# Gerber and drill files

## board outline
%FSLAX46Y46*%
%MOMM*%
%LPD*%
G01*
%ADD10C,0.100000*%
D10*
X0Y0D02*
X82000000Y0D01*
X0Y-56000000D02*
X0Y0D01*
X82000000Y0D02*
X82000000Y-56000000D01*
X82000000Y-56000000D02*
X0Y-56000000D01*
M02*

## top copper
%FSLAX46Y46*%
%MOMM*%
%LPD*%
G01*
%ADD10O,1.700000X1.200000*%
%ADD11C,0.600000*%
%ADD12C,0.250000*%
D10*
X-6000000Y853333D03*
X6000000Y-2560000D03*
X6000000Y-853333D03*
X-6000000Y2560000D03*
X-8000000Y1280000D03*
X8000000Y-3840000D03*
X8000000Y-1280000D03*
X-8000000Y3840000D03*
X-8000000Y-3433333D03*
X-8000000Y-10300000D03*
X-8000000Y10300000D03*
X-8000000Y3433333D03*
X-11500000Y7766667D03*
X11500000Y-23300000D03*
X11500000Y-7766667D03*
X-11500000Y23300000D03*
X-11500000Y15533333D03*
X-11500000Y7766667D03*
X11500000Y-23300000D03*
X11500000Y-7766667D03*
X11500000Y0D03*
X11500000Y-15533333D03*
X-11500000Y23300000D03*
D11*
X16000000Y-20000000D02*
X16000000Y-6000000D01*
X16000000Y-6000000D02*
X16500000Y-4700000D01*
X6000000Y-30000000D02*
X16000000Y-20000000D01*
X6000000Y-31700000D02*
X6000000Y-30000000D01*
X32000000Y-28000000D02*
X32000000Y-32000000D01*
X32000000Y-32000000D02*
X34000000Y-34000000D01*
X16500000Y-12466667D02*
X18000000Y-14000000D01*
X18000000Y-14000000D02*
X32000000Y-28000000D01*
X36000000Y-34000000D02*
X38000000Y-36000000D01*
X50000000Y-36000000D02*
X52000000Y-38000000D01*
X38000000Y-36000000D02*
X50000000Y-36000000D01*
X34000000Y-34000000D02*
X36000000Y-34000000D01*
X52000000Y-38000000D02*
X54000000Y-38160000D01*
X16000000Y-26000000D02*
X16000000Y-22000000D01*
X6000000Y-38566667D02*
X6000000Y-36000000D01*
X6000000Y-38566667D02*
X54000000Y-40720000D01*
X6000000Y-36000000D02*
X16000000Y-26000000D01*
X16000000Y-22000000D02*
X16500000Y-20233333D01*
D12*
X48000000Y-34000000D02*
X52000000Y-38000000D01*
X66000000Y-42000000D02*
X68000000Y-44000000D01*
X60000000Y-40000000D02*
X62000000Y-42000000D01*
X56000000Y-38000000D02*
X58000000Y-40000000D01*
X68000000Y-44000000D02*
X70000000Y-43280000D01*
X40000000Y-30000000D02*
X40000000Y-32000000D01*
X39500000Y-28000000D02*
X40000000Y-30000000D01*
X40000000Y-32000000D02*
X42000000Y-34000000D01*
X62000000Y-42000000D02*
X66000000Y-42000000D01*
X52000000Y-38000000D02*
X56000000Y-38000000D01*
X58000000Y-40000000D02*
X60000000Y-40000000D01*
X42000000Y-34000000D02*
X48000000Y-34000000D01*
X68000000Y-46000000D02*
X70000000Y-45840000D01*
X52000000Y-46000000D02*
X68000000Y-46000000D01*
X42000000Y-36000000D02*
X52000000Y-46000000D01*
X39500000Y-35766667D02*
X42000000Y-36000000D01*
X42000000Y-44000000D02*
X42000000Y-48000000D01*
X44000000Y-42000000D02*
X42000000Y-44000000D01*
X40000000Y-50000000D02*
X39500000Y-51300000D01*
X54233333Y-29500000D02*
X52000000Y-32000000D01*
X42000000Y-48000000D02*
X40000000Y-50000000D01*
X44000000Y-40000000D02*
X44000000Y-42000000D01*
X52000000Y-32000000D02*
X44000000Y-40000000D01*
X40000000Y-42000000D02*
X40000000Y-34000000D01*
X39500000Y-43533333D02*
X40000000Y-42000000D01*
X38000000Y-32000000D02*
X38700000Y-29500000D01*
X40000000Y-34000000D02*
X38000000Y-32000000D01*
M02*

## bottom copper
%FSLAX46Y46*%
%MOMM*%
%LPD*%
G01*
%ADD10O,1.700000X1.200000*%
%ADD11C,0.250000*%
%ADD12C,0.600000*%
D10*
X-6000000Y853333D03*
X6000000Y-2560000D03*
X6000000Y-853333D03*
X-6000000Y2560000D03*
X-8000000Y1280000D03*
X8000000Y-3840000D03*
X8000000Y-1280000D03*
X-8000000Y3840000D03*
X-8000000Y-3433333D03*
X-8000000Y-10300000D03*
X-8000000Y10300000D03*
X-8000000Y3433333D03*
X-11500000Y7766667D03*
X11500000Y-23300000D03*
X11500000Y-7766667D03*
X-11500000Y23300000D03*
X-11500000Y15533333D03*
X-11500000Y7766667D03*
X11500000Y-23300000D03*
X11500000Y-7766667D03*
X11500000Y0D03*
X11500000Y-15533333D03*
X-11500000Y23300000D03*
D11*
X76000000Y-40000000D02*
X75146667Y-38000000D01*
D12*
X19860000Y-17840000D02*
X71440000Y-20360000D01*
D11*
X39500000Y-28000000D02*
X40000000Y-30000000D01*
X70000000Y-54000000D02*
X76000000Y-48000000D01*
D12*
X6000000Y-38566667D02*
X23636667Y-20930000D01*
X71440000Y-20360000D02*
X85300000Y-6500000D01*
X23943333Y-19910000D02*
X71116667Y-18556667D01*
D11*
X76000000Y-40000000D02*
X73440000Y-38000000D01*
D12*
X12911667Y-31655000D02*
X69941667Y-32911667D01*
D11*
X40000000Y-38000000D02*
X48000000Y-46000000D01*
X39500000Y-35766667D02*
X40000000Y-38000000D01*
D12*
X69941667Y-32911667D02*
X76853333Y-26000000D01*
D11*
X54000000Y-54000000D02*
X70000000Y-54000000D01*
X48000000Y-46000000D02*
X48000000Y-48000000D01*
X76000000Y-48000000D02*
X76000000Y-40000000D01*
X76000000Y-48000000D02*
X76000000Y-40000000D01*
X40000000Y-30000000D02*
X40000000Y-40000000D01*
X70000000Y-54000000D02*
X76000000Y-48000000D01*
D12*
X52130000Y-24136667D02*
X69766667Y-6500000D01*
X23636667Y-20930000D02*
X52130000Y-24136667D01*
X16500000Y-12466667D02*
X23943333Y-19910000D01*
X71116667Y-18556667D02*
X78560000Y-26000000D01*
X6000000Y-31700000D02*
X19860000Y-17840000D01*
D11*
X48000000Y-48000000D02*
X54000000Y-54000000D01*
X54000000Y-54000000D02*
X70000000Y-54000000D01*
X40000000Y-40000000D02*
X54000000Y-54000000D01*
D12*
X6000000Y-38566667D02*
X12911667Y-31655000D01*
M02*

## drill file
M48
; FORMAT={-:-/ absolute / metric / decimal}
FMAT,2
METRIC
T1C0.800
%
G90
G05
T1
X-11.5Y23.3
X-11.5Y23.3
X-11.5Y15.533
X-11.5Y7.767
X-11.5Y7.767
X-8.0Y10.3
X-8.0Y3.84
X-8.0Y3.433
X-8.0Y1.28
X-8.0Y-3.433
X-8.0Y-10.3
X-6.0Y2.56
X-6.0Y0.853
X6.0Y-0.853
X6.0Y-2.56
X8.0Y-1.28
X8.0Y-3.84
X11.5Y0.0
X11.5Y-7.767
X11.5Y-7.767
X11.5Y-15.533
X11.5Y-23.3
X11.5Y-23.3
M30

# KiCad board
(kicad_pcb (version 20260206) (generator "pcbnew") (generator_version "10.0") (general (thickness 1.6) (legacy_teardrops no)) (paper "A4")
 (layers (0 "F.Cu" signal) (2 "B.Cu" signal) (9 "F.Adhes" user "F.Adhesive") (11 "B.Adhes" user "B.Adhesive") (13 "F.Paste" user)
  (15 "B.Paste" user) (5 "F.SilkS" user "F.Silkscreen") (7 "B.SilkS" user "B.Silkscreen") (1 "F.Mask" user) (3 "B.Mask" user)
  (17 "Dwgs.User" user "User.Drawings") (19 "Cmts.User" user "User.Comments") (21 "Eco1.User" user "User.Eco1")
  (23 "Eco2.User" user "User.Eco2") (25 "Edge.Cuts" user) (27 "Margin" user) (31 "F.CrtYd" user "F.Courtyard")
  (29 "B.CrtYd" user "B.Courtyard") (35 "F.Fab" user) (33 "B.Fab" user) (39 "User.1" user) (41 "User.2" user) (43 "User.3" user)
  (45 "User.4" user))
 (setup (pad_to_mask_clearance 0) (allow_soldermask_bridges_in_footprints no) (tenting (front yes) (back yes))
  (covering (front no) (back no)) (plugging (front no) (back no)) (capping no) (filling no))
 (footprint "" (layer "F.Cu") (at 76 32 90)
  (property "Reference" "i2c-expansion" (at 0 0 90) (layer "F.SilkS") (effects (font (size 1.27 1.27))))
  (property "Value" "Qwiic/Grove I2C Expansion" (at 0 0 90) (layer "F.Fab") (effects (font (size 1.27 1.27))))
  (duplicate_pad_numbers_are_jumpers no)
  (pad "GND" thru_hole oval (at 32.853333 -82) (size 1.7 1.2) (drill 0.8) (layers "*.Cu") (remove_unused_layers no) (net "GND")
   (thermal_bridge_angle 45))
  (pad "SCL" thru_hole oval (at 29.44 -70) (size 1.7 1.2) (drill 0.8) (layers "*.Cu") (remove_unused_layers no) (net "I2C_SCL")
   (thermal_bridge_angle 45))
  (pad "SDA" thru_hole oval (at 31.146667 -70) (size 1.7 1.2) (drill 0.8) (layers "*.Cu") (remove_unused_layers no) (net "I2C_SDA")
   (thermal_bridge_angle 45))
  (pad "VCC" thru_hole oval (at 34.56 -82) (size 1.7 1.2) (drill 0.8) (layers "*.Cu") (remove_unused_layers no) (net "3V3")
   (thermal_bridge_angle 45)))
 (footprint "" (layer "F.Cu") (at 62 42)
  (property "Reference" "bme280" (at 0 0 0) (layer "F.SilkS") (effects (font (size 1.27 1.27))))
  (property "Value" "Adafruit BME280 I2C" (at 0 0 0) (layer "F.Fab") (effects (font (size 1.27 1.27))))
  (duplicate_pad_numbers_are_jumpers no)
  (pad "GND" thru_hole oval (at -70 -43.28) (size 1.7 1.2) (drill 0.8) (layers "*.Cu") (remove_unused_layers no) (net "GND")
   (thermal_bridge_angle 45))
  (pad "SCL" thru_hole oval (at -54 -38.16) (size 1.7 1.2) (drill 0.8) (layers "*.Cu") (remove_unused_layers no) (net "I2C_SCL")
   (thermal_bridge_angle 45))
  (pad "SDA" thru_hole oval (at -54 -40.72) (size 1.7 1.2) (drill 0.8) (layers "*.Cu") (remove_unused_layers no) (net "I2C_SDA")
   (thermal_bridge_angle 45))
  (pad "VCC" thru_hole oval (at -70 -45.84) (size 1.7 1.2) (drill 0.8) (layers "*.Cu") (remove_unused_layers no) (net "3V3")
   (thermal_bridge_angle 45)))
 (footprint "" (layer "F.Cu") (at 14 42)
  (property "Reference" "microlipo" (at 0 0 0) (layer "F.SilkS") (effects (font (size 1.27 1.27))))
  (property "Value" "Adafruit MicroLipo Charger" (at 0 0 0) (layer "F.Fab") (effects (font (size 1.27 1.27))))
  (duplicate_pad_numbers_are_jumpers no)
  (pad "B+" thru_hole oval (at -22 -38.566667) (size 1.7 1.2) (drill 0.8) (layers "*.Cu") (remove_unused_layers no)
   (thermal_bridge_angle 45))
  (pad "B-" thru_hole oval (at -22 -31.7) (size 1.7 1.2) (drill 0.8) (layers "*.Cu") (remove_unused_layers no) (thermal_bridge_angle 45))
  (pad "OUT+" thru_hole oval (at -22 -52.3) (size 1.7 1.2) (drill 0.8) (layers "*.Cu") (remove_unused_layers no) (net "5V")
   (thermal_bridge_angle 45))
  (pad "OUT-" thru_hole oval (at -22 -45.433333) (size 1.7 1.2) (drill 0.8) (layers "*.Cu") (remove_unused_layers no) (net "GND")
   (thermal_bridge_angle 45)))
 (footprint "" (layer "F.Cu") (at 62 18 90)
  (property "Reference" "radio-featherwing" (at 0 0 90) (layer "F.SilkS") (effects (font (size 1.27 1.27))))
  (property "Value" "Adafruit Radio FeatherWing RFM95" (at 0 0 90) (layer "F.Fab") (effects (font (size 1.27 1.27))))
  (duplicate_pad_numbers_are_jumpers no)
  (pad "GND" thru_hole oval (at 25.766667 -73.5) (size 1.7 1.2) (drill 0.8) (layers "*.Cu") (remove_unused_layers no) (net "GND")
   (thermal_bridge_angle 45))
  (pad "RX" thru_hole oval (at -5.3 -50.5) (size 1.7 1.2) (drill 0.8) (layers "*.Cu") (remove_unused_layers no) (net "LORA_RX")
   (thermal_bridge_angle 45))
  (pad "TX" thru_hole oval (at 10.233333 -50.5) (size 1.7 1.2) (drill 0.8) (layers "*.Cu") (remove_unused_layers no) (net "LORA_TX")
   (thermal_bridge_angle 45))
  (pad "VCC" thru_hole oval (at 41.3 -73.5) (size 1.7 1.2) (drill 0.8) (layers "*.Cu") (remove_unused_layers no) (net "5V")
   (thermal_bridge_angle 45)))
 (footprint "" (layer "F.Cu") (at 28 28)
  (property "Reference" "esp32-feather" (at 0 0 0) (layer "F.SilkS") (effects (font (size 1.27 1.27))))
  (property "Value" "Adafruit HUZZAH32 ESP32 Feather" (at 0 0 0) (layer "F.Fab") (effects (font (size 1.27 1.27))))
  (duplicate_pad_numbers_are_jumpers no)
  (pad "3V3" thru_hole oval (at -39.5 -43.533333) (size 1.7 1.2) (drill 0.8) (layers "*.Cu") (remove_unused_layers no) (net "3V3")
   (thermal_bridge_angle 45))
  (pad "GND" thru_hole oval (at -39.5 -35.766667) (size 1.7 1.2) (drill 0.8) (layers "*.Cu") (remove_unused_layers no) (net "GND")
   (thermal_bridge_angle 45))
  (pad "RX" thru_hole oval (at -16.5 -4.7) (size 1.7 1.2) (drill 0.8) (layers "*.Cu") (remove_unused_layers no) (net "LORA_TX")
   (thermal_bridge_angle 45))
  (pad "SCL" thru_hole oval (at -16.5 -20.233333) (size 1.7 1.2) (drill 0.8) (layers "*.Cu") (remove_unused_layers no) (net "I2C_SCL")
   (thermal_bridge_angle 45))
  (pad "SDA" thru_hole oval (at -16.5 -28) (size 1.7 1.2) (drill 0.8) (layers "*.Cu") (remove_unused_layers no) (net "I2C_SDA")
   (thermal_bridge_angle 45))
  (pad "TX" thru_hole oval (at -16.5 -12.466667) (size 1.7 1.2) (drill 0.8) (layers "*.Cu") (remove_unused_layers no) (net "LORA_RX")
   (thermal_bridge_angle 45))
  (pad "VIN" thru_hole oval (at -39.5 -51.3) (size 1.7 1.2) (drill 0.8) (layers "*.Cu") (remove_unused_layers no) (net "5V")
   (thermal_bridge_angle 45)))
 (gr_line (start 0 0) (end 82 0) (stroke (width 0.1) (type default)) (layer "Edge.Cuts"))
 (gr_line (start 0 56) (end 0 0) (stroke (width 0.1) (type default)) (layer "Edge.Cuts"))
 (gr_line (start 82 0) (end 82 56) (stroke (width 0.1) (type default)) (layer "Edge.Cuts"))
 (gr_line (start 82 56) (end 0 56) (stroke (width 0.1) (type default)) (layer "Edge.Cuts"))
 (segment (start 16 20) (end 16 6) (width 0.6) (layer "F.Cu") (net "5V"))
 (segment (start 16 6) (end 16.5 4.7) (width 0.6) (layer "F.Cu") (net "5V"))
 (segment (start 6 30) (end 16 20) (width 0.6) (layer "F.Cu") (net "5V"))
 (segment (start 6 31.7) (end 6 30) (width 0.6) (layer "F.Cu") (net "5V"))
 (segment (start 32 28) (end 32 32) (width 0.6) (layer "F.Cu") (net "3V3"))
 (segment (start 32 32) (end 34 34) (width 0.6) (layer "F.Cu") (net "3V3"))
 (segment (start 16.5 12.466667) (end 18 14) (width 0.6) (layer "F.Cu") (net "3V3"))
 (segment (start 18 14) (end 32 28) (width 0.6) (layer "F.Cu") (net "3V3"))
 (segment (start 36 34) (end 38 36) (width 0.6) (layer "F.Cu") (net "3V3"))
 (segment (start 50 36) (end 52 38) (width 0.6) (layer "F.Cu") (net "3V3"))
 (segment (start 38 36) (end 50 36) (width 0.6) (layer "F.Cu") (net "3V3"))
 (segment (start 34 34) (end 36 34) (width 0.6) (layer "F.Cu") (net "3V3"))
 (segment (start 52 38) (end 54 38.16) (width 0.6) (layer "F.Cu") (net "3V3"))
 (segment (start 16 26) (end 16 22) (width 0.6) (layer "F.Cu") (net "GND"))
 (segment (start 6 38.566667) (end 6 36) (width 0.6) (layer "F.Cu") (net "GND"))
 (segment (start 6 38.566667) (end 54 40.72) (width 0.6) (layer "F.Cu") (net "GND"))
 (segment (start 6 36) (end 16 26) (width 0.6) (layer "F.Cu") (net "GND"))
 (segment (start 16 22) (end 16.5 20.233333) (width 0.6) (layer "F.Cu") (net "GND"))
 (segment (start 48 34) (end 52 38) (width 0.25) (layer "F.Cu") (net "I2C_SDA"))
 (segment (start 66 42) (end 68 44) (width 0.25) (layer "F.Cu") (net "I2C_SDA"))
 (segment (start 60 40) (end 62 42) (width 0.25) (layer "F.Cu") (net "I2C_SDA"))
 (segment (start 56 38) (end 58 40) (width 0.25) (layer "F.Cu") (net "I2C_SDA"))
 (segment (start 68 44) (end 70 43.28) (width 0.25) (layer "F.Cu") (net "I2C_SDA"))
 (segment (start 40 30) (end 40 32) (width 0.25) (layer "F.Cu") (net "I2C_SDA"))
 (segment (start 39.5 28) (end 40 30) (width 0.25) (layer "F.Cu") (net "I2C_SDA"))
 (segment (start 40 32) (end 42 34) (width 0.25) (layer "F.Cu") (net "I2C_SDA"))
 (segment (start 62 42) (end 66 42) (width 0.25) (layer "F.Cu") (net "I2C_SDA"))
 (segment (start 52 38) (end 56 38) (width 0.25) (layer "F.Cu") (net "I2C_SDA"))
 (segment (start 58 40) (end 60 40) (width 0.25) (layer "F.Cu") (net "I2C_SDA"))
 (segment (start 42 34) (end 48 34) (width 0.25) (layer "F.Cu") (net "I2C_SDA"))
 (segment (start 68 46) (end 70 45.84) (width 0.25) (layer "F.Cu") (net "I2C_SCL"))
 (segment (start 52 46) (end 68 46) (width 0.25) (layer "F.Cu") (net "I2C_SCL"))
 (segment (start 42 36) (end 52 46) (width 0.25) (layer "F.Cu") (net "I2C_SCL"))
 (segment (start 39.5 35.766667) (end 42 36) (width 0.25) (layer "F.Cu") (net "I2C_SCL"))
 (segment (start 76 40) (end 75.146667 38) (width 0.25) (layer "B.Cu") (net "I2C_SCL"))
 (segment (start 19.86 17.84) (end 71.44 20.36) (width 0.6) (layer "B.Cu") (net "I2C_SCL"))
 (segment (start 39.5 28) (end 40 30) (width 0.25) (layer "B.Cu") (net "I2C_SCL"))
 (segment (start 70 54) (end 76 48) (width 0.25) (layer "B.Cu") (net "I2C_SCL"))
 (segment (start 6 38.566667) (end 23.636667 20.93) (width 0.6) (layer "B.Cu") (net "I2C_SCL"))
 (segment (start 71.44 20.36) (end 85.3 6.5) (width 0.6) (layer "B.Cu") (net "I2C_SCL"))
 (segment (start 23.943333 19.91) (end 71.116667 18.556667) (width 0.6) (layer "B.Cu") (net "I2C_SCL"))
 (segment (start 76 40) (end 73.44 38) (width 0.25) (layer "B.Cu") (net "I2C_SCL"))
 (segment (start 12.911667 31.655) (end 69.941667 32.911667) (width 0.6) (layer "B.Cu") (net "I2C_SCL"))
 (segment (start 40 38) (end 48 46) (width 0.25) (layer "B.Cu") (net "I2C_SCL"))
 (segment (start 39.5 35.766667) (end 40 38) (width 0.25) (layer "B.Cu") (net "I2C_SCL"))
 (segment (start 69.941667 32.911667) (end 76.853333 26) (width 0.6) (layer "B.Cu") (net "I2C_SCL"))
 (segment (start 54 54) (end 70 54) (width 0.25) (layer "B.Cu") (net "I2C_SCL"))
 (segment (start 48 46) (end 48 48) (width 0.25) (layer "B.Cu") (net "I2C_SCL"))
 (segment (start 76 48) (end 76 40) (width 0.25) (layer "B.Cu") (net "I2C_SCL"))
 (segment (start 76 48) (end 76 40) (width 0.25) (layer "B.Cu") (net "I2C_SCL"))
 (segment (start 40 30) (end 40 40) (width 0.25) (layer "B.Cu") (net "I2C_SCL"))
 (segment (start 70 54) (end 76 48) (width 0.25) (layer "B.Cu") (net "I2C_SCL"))
 (segment (start 52.13 24.136667) (end 69.766667 6.5) (width 0.6) (layer "B.Cu") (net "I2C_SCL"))
 (segment (start 23.636667 20.93) (end 52.13 24.136667) (width 0.6) (layer "B.Cu") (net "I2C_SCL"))
 (segment (start 16.5 12.466667) (end 23.943333 19.91) (width 0.6) (layer "B.Cu") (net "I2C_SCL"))
 (segment (start 71.116667 18.556667) (end 78.56 26) (width 0.6) (layer "B.Cu") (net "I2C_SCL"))
 (segment (start 6 31.7) (end 19.86 17.84) (width 0.6) (layer "B.Cu") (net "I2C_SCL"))
 (segment (start 48 48) (end 54 54) (width 0.25) (layer "B.Cu") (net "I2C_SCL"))
 (segment (start 54 54) (end 70 54) (width 0.25) (layer "B.Cu") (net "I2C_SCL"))
 (segment (start 40 40) (end 54 54) (width 0.25) (layer "B.Cu") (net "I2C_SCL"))
 (segment (start 6 38.566667) (end 12.911667 31.655) (width 0.6) (layer "B.Cu") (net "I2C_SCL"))
 (segment (start 42 44) (end 42 48) (width 0.25) (layer "F.Cu") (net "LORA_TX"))
 (segment (start 44 42) (end 42 44) (width 0.25) (layer "F.Cu") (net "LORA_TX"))
 (segment (start 40 50) (end 39.5 51.3) (width 0.25) (layer "F.Cu") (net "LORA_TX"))
 (segment (start 54.233333 29.5) (end 52 32) (width 0.25) (layer "F.Cu") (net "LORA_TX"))
 (segment (start 42 48) (end 40 50) (width 0.25) (layer "F.Cu") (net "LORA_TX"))
 (segment (start 44 40) (end 44 42) (width 0.25) (layer "F.Cu") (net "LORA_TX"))
 (segment (start 52 32) (end 44 40) (width 0.25) (layer "F.Cu") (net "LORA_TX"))
 (segment (start 40 42) (end 40 34) (width 0.25) (layer "F.Cu") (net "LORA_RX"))
 (segment (start 39.5 43.533333) (end 40 42) (width 0.25) (layer "F.Cu") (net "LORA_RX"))
 (segment (start 38 32) (end 38.7 29.5) (width 0.25) (layer "F.Cu") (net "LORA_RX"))
 (segment (start 40 34) (end 38 32) (width 0.25) (layer "F.Cu") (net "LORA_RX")))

